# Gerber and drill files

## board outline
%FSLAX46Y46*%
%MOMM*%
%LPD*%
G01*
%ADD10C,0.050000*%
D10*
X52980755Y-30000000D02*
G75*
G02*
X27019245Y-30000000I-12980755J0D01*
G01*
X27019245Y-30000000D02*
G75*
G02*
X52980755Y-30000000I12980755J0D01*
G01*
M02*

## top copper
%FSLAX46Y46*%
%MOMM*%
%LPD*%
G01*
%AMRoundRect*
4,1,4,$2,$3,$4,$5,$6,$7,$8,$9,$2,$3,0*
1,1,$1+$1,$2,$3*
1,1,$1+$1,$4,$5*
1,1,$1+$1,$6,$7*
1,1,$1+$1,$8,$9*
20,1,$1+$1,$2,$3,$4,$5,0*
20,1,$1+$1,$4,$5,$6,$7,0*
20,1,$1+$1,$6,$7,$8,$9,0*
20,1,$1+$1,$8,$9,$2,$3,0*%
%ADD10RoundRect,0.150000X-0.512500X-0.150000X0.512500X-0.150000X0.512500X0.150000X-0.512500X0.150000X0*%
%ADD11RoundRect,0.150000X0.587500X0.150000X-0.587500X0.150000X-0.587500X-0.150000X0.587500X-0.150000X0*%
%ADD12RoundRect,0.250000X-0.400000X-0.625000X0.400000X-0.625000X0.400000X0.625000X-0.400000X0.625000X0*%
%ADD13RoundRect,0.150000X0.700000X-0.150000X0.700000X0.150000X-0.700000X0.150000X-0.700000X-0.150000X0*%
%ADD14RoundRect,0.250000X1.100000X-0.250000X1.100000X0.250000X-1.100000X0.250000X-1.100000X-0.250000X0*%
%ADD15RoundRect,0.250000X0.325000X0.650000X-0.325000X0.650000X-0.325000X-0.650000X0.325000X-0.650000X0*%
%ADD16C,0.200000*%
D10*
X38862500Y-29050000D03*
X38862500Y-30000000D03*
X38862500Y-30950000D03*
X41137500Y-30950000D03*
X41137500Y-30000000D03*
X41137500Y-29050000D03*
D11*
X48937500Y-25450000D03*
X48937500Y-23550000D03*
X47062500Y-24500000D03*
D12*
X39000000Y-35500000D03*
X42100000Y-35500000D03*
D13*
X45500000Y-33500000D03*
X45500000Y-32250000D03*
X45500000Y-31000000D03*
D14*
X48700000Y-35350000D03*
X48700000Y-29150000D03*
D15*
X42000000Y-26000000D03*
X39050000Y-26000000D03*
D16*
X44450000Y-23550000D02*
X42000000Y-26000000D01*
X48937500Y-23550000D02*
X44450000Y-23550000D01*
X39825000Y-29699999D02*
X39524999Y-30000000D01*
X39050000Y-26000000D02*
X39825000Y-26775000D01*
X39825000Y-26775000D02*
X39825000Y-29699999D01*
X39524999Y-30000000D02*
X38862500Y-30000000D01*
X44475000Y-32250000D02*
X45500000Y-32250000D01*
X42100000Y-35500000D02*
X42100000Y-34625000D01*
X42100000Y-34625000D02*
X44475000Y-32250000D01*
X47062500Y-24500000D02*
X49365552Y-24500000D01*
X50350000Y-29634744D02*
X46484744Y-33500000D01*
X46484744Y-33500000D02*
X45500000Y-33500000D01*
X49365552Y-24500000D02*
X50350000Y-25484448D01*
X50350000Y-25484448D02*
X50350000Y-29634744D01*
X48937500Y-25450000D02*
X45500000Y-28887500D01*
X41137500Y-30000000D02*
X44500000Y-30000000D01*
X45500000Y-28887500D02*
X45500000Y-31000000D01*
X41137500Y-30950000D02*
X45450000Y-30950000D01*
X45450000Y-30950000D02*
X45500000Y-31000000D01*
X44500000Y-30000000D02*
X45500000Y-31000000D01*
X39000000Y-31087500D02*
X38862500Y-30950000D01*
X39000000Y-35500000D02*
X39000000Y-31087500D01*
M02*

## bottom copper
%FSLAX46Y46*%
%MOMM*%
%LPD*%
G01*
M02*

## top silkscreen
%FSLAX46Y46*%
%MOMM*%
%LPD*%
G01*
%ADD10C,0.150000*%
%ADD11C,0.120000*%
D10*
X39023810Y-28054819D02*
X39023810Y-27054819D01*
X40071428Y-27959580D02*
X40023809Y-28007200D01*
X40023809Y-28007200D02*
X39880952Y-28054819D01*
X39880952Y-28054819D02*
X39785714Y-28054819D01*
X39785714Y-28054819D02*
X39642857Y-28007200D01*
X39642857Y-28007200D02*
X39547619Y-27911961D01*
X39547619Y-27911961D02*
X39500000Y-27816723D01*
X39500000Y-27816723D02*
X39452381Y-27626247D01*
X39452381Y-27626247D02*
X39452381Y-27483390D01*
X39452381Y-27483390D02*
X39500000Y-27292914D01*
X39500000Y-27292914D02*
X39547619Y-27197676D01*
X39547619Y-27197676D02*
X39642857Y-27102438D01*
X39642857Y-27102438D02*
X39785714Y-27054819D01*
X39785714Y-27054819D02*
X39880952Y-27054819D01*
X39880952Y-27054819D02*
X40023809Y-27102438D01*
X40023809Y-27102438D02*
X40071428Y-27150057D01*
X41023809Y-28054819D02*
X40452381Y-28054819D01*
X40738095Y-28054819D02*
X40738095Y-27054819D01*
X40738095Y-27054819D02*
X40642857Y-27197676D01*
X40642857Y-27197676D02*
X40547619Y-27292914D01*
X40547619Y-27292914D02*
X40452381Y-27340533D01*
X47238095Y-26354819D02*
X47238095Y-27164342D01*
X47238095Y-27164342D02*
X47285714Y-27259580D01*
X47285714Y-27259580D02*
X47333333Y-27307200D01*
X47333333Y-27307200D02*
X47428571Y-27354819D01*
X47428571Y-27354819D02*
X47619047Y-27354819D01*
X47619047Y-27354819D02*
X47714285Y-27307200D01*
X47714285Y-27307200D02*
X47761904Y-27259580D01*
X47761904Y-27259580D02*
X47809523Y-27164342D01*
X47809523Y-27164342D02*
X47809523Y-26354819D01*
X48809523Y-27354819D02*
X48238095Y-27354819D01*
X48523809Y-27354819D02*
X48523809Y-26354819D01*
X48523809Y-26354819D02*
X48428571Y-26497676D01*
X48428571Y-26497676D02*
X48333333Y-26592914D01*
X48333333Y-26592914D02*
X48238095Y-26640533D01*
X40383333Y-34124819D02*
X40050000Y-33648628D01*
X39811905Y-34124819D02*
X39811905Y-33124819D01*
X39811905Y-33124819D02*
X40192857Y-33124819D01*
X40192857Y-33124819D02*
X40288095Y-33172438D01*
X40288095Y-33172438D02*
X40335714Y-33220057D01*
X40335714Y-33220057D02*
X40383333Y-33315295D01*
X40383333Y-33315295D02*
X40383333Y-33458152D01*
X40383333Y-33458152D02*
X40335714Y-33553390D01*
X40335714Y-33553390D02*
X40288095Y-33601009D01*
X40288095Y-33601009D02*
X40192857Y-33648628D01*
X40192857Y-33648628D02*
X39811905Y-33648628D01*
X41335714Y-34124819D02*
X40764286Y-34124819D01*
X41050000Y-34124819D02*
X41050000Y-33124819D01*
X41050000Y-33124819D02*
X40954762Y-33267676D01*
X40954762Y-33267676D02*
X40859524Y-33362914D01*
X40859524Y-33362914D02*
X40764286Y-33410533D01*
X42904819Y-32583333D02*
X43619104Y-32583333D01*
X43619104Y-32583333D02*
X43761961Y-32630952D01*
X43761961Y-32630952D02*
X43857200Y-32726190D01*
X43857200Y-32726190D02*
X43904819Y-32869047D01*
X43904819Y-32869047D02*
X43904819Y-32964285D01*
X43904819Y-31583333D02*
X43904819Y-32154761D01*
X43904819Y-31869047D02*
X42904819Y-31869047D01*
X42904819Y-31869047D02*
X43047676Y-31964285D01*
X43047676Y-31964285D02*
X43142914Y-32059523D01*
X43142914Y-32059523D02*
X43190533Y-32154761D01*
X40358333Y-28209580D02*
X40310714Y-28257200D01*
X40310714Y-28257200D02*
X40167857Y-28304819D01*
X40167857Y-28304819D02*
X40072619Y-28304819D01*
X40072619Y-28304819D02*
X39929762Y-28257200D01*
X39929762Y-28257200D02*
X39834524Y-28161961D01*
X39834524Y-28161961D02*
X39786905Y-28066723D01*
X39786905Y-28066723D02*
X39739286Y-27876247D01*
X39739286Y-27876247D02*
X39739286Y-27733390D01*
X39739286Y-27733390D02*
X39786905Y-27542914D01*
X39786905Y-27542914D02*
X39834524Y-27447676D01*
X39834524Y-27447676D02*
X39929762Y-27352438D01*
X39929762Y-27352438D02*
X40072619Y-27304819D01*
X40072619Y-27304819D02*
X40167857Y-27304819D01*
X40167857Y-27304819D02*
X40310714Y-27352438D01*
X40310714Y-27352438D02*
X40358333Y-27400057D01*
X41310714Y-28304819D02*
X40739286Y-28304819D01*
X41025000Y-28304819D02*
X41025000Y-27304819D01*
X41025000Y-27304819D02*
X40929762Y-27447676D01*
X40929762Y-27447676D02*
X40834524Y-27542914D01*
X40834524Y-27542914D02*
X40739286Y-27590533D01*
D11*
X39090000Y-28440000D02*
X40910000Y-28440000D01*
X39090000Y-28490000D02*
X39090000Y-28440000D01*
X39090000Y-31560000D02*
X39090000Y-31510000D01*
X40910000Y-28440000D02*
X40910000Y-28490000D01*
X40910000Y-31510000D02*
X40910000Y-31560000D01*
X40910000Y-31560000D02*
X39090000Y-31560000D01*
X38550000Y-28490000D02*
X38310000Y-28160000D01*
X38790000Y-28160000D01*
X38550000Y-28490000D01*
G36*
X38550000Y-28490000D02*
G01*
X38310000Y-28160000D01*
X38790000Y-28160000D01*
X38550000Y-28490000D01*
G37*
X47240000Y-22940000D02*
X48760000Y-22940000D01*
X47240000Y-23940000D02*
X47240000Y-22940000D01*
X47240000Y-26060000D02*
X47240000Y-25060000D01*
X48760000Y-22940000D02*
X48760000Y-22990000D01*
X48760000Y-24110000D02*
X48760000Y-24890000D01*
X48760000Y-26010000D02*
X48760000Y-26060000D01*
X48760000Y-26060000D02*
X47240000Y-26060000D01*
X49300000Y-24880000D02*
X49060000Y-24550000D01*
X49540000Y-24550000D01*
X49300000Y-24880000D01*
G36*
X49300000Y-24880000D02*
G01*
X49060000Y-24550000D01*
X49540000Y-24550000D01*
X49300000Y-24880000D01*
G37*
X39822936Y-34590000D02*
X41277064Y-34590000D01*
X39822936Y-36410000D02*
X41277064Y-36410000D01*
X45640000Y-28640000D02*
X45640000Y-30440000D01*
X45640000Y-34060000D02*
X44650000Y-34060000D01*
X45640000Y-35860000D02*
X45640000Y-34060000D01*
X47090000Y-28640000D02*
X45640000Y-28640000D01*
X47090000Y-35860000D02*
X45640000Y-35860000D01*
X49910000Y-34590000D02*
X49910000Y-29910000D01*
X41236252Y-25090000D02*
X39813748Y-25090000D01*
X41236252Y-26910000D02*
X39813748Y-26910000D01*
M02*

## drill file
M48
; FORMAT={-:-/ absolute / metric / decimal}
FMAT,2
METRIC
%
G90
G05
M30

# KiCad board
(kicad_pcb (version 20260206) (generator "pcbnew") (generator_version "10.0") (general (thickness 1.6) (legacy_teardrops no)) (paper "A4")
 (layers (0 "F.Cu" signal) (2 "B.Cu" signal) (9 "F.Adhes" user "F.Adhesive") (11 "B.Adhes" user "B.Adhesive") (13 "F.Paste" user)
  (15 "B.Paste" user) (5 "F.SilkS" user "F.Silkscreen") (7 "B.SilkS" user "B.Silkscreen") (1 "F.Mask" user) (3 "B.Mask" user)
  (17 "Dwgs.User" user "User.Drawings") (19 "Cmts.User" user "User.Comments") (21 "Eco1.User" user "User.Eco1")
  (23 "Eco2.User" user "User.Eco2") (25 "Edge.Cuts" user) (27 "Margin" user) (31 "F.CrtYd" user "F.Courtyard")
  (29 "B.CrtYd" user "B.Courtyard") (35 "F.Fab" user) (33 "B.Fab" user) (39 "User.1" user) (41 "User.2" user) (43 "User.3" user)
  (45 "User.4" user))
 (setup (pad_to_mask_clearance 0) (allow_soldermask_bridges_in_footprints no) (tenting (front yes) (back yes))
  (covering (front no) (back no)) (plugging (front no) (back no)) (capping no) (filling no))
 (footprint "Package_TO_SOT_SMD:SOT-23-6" (layer "F.Cu") (at 40 30)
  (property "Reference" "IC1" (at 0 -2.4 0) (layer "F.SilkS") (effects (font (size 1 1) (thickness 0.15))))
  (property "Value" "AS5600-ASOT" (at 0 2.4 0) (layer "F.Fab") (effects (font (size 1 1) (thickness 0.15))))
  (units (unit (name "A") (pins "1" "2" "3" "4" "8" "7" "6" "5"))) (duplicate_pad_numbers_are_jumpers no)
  (fp_line (start -0.91 -1.56) (end 0.91 -1.56) (stroke (width 0.12) (type solid)) (layer "F.SilkS"))
  (fp_line (start -0.91 -1.51) (end -0.91 -1.56) (stroke (width 0.12) (type solid)) (layer "F.SilkS"))
  (fp_line (start -0.91 1.56) (end -0.91 1.51) (stroke (width 0.12) (type solid)) (layer "F.SilkS"))
  (fp_line (start 0.91 -1.56) (end 0.91 -1.51) (stroke (width 0.12) (type solid)) (layer "F.SilkS"))
  (fp_line (start 0.91 1.51) (end 0.91 1.56) (stroke (width 0.12) (type solid)) (layer "F.SilkS"))
  (fp_line (start 0.91 1.56) (end -0.91 1.56) (stroke (width 0.12) (type solid)) (layer "F.SilkS"))
  (fp_poly (pts (xy -1.45 -1.51) (xy -1.69 -1.84) (xy -1.21 -1.84)) (stroke (width 0.12) (type solid)) (fill yes) (layer "F.SilkS"))
  (pad "1" smd roundrect (at -1.1375 -0.95) (size 1.325 0.6) (layers "F.Cu" "F.Mask" "F.Paste") (roundrect_rratio 0.25)
   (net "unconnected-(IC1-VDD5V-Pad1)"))
  (pad "2" smd roundrect (at -1.1375 0) (size 1.325 0.6) (layers "F.Cu" "F.Mask" "F.Paste") (roundrect_rratio 0.25) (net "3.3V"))
  (pad "3" smd roundrect (at -1.1375 0.95) (size 1.325 0.6) (layers "F.Cu" "F.Mask" "F.Paste") (roundrect_rratio 0.25) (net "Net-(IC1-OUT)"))
  (pad "4" smd roundrect (at 1.1375 0.95) (size 1.325 0.6) (layers "F.Cu" "F.Mask" "F.Paste") (roundrect_rratio 0.25) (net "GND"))
  (pad "5" smd roundrect (at 1.1375 0) (size 1.325 0.6) (layers "F.Cu" "F.Mask" "F.Paste") (roundrect_rratio 0.25) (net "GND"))
  (pad "6" smd roundrect (at 1.1375 -0.95) (size 1.325 0.6) (layers "F.Cu" "F.Mask" "F.Paste") (roundrect_rratio 0.25)
   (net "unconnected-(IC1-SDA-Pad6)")))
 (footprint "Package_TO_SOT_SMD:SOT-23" (layer "F.Cu") (at 48 24.5 180)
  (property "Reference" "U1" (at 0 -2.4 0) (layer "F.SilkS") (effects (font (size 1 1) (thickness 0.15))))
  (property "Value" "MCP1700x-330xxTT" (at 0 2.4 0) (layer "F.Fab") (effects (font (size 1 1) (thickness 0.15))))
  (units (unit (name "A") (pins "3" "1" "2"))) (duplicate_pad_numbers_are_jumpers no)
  (fp_line (start 0.76 1.56) (end -0.76 1.56) (stroke (width 0.12) (type solid)) (layer "F.SilkS"))
  (fp_line (start 0.76 0.56) (end 0.76 1.56) (stroke (width 0.12) (type solid)) (layer "F.SilkS"))
  (fp_line (start 0.76 -1.56) (end 0.76 -0.56) (stroke (width 0.12) (type solid)) (layer "F.SilkS"))
  (fp_line (start -0.76 1.56) (end -0.76 1.51) (stroke (width 0.12) (type solid)) (layer "F.SilkS"))
  (fp_line (start -0.76 0.39) (end -0.76 -0.39) (stroke (width 0.12) (type solid)) (layer "F.SilkS"))
  (fp_line (start -0.76 -1.51) (end -0.76 -1.56) (stroke (width 0.12) (type solid)) (layer "F.SilkS"))
  (fp_line (start -0.76 -1.56) (end 0.76 -1.56) (stroke (width 0.12) (type solid)) (layer "F.SilkS"))
  (fp_poly (pts (xy -1.3 -0.38) (xy -1.06 -0.05) (xy -1.54 -0.05)) (stroke (width 0.12) (type solid)) (fill yes) (layer "F.SilkS"))
  (pad "1" smd roundrect (at -0.9375 -0.95 180) (size 1.475 0.6) (layers "F.Cu" "F.Mask" "F.Paste") (roundrect_rratio 0.25) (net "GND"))
  (pad "2" smd roundrect (at -0.9375 0.95 180) (size 1.475 0.6) (layers "F.Cu" "F.Mask" "F.Paste") (roundrect_rratio 0.25)
   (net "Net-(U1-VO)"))
  (pad "3" smd roundrect (at 0.9375 0 180) (size 1.475 0.6) (layers "F.Cu" "F.Mask" "F.Paste") (roundrect_rratio 0.25) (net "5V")))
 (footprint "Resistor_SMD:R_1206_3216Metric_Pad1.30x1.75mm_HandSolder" (layer "F.Cu") (at 40.55 35.5)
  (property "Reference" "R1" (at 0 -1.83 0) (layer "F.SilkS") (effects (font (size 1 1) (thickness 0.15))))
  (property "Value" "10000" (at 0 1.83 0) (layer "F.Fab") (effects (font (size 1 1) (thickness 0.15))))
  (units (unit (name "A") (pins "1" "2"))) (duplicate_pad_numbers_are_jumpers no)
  (fp_line (start -0.727064 -0.91) (end 0.727064 -0.91) (stroke (width 0.12) (type solid)) (layer "F.SilkS"))
  (fp_line (start -0.727064 0.91) (end 0.727064 0.91) (stroke (width 0.12) (type solid)) (layer "F.SilkS"))
  (pad "1" smd roundrect (at -1.55 0) (size 1.3 1.75) (layers "F.Cu" "F.Mask" "F.Paste") (roundrect_rratio 0.192308) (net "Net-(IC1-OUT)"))
  (pad "2" smd roundrect (at 1.55 0) (size 1.3 1.75) (layers "F.Cu" "F.Mask" "F.Paste") (roundrect_rratio 0.192308) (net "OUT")))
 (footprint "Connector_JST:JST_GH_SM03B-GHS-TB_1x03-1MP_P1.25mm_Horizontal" (layer "F.Cu") (at 47.35 32.25 90)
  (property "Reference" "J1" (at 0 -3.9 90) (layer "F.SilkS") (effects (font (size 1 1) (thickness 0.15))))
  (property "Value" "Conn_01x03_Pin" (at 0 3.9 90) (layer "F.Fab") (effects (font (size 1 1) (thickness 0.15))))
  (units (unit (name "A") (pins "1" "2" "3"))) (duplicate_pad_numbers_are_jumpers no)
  (fp_line (start 3.61 -1.71) (end 1.81 -1.71) (stroke (width 0.12) (type solid)) (layer "F.SilkS"))
  (fp_line (start -1.81 -1.71) (end -1.81 -2.7) (stroke (width 0.12) (type solid)) (layer "F.SilkS"))
  (fp_line (start -3.61 -1.71) (end -1.81 -1.71) (stroke (width 0.12) (type solid)) (layer "F.SilkS"))
  (fp_line (start 3.61 -0.26) (end 3.61 -1.71) (stroke (width 0.12) (type solid)) (layer "F.SilkS"))
  (fp_line (start -3.61 -0.26) (end -3.61 -1.71) (stroke (width 0.12) (type solid)) (layer "F.SilkS"))
  (fp_line (start -2.34 2.56) (end 2.34 2.56) (stroke (width 0.12) (type solid)) (layer "F.SilkS"))
  (pad "1" smd roundrect (at -1.25 -1.85 90) (size 0.6 1.7) (layers "F.Cu" "F.Mask" "F.Paste") (roundrect_rratio 0.25) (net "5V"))
  (pad "2" smd roundrect (at 0 -1.85 90) (size 0.6 1.7) (layers "F.Cu" "F.Mask" "F.Paste") (roundrect_rratio 0.25) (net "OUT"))
  (pad "3" smd roundrect (at 1.25 -1.85 90) (size 0.6 1.7) (layers "F.Cu" "F.Mask" "F.Paste") (roundrect_rratio 0.25) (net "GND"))
  (pad "MP" smd roundrect (at -3.1 1.35 90) (size 1 2.7) (layers "F.Cu" "F.Mask" "F.Paste") (roundrect_rratio 0.25))
  (pad "MP" smd roundrect (at 3.1 1.35 90) (size 1 2.7) (layers "F.Cu" "F.Mask" "F.Paste") (roundrect_rratio 0.25)))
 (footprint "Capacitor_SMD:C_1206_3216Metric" (layer "F.Cu") (at 40.525 26 180)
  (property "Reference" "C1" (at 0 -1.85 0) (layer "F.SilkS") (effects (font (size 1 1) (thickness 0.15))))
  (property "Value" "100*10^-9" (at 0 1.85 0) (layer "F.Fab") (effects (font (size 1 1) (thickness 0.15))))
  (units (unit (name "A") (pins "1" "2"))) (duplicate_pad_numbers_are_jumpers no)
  (fp_line (start -0.711252 0.91) (end 0.711252 0.91) (stroke (width 0.12) (type solid)) (layer "F.SilkS"))
  (fp_line (start -0.711252 -0.91) (end 0.711252 -0.91) (stroke (width 0.12) (type solid)) (layer "F.SilkS"))
  (pad "1" smd roundrect (at -1.475 0 180) (size 1.15 1.8) (layers "F.Cu" "F.Mask" "F.Paste") (roundrect_rratio 0.217391)
   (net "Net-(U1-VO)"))
  (pad "2" smd roundrect (at 1.475 0 180) (size 1.15 1.8) (layers "F.Cu" "F.Mask" "F.Paste") (roundrect_rratio 0.217391) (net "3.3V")))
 (gr_circle (center 40 30) (end 52.5 33.5) (stroke (width 0.05) (type default)) (fill no) (layer "Edge.Cuts"))
 (segment (start 44.45 23.55) (end 42 26) (width 0.2) (layer "F.Cu") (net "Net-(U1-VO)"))
 (segment (start 48.9375 23.55) (end 44.45 23.55) (width 0.2) (layer "F.Cu") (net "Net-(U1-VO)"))
 (segment (start 39.825 29.699999) (end 39.524999 30) (width 0.2) (layer "F.Cu") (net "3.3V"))
 (segment (start 39.05 26) (end 39.825 26.775) (width 0.2) (layer "F.Cu") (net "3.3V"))
 (segment (start 39.825 26.775) (end 39.825 29.699999) (width 0.2) (layer "F.Cu") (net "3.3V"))
 (segment (start 39.524999 30) (end 38.8625 30) (width 0.2) (layer "F.Cu") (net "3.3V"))
 (segment (start 44.475 32.25) (end 45.5 32.25) (width 0.2) (layer "F.Cu") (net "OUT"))
 (segment (start 42.1 35.5) (end 42.1 34.625) (width 0.2) (layer "F.Cu") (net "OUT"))
 (segment (start 42.1 34.625) (end 44.475 32.25) (width 0.2) (layer "F.Cu") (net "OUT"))
 (segment (start 47.0625 24.5) (end 49.365552 24.5) (width 0.2) (layer "F.Cu") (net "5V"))
 (segment (start 50.35 29.634744) (end 46.484744 33.5) (width 0.2) (layer "F.Cu") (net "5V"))
 (segment (start 46.484744 33.5) (end 45.5 33.5) (width 0.2) (layer "F.Cu") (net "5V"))
 (segment (start 49.365552 24.5) (end 50.35 25.484448) (width 0.2) (layer "F.Cu") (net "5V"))
 (segment (start 50.35 25.484448) (end 50.35 29.634744) (width 0.2) (layer "F.Cu") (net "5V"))
 (segment (start 48.9375 25.45) (end 45.5 28.8875) (width 0.2) (layer "F.Cu") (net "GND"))
 (segment (start 41.1375 30) (end 44.5 30) (width 0.2) (layer "F.Cu") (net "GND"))
 (segment (start 45.5 28.8875) (end 45.5 31) (width 0.2) (layer "F.Cu") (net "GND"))
 (segment (start 41.1375 30.95) (end 45.45 30.95) (width 0.2) (layer "F.Cu") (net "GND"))
 (segment (start 45.45 30.95) (end 45.5 31) (width 0.2) (layer "F.Cu") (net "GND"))
 (segment (start 44.5 30) (end 45.5 31) (width 0.2) (layer "F.Cu") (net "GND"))
 (segment (start 39 31.0875) (end 38.8625 30.95) (width 0.2) (layer "F.Cu") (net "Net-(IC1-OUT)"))
 (segment (start 39 35.5) (end 39 31.0875) (width 0.2) (layer "F.Cu") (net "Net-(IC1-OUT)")))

